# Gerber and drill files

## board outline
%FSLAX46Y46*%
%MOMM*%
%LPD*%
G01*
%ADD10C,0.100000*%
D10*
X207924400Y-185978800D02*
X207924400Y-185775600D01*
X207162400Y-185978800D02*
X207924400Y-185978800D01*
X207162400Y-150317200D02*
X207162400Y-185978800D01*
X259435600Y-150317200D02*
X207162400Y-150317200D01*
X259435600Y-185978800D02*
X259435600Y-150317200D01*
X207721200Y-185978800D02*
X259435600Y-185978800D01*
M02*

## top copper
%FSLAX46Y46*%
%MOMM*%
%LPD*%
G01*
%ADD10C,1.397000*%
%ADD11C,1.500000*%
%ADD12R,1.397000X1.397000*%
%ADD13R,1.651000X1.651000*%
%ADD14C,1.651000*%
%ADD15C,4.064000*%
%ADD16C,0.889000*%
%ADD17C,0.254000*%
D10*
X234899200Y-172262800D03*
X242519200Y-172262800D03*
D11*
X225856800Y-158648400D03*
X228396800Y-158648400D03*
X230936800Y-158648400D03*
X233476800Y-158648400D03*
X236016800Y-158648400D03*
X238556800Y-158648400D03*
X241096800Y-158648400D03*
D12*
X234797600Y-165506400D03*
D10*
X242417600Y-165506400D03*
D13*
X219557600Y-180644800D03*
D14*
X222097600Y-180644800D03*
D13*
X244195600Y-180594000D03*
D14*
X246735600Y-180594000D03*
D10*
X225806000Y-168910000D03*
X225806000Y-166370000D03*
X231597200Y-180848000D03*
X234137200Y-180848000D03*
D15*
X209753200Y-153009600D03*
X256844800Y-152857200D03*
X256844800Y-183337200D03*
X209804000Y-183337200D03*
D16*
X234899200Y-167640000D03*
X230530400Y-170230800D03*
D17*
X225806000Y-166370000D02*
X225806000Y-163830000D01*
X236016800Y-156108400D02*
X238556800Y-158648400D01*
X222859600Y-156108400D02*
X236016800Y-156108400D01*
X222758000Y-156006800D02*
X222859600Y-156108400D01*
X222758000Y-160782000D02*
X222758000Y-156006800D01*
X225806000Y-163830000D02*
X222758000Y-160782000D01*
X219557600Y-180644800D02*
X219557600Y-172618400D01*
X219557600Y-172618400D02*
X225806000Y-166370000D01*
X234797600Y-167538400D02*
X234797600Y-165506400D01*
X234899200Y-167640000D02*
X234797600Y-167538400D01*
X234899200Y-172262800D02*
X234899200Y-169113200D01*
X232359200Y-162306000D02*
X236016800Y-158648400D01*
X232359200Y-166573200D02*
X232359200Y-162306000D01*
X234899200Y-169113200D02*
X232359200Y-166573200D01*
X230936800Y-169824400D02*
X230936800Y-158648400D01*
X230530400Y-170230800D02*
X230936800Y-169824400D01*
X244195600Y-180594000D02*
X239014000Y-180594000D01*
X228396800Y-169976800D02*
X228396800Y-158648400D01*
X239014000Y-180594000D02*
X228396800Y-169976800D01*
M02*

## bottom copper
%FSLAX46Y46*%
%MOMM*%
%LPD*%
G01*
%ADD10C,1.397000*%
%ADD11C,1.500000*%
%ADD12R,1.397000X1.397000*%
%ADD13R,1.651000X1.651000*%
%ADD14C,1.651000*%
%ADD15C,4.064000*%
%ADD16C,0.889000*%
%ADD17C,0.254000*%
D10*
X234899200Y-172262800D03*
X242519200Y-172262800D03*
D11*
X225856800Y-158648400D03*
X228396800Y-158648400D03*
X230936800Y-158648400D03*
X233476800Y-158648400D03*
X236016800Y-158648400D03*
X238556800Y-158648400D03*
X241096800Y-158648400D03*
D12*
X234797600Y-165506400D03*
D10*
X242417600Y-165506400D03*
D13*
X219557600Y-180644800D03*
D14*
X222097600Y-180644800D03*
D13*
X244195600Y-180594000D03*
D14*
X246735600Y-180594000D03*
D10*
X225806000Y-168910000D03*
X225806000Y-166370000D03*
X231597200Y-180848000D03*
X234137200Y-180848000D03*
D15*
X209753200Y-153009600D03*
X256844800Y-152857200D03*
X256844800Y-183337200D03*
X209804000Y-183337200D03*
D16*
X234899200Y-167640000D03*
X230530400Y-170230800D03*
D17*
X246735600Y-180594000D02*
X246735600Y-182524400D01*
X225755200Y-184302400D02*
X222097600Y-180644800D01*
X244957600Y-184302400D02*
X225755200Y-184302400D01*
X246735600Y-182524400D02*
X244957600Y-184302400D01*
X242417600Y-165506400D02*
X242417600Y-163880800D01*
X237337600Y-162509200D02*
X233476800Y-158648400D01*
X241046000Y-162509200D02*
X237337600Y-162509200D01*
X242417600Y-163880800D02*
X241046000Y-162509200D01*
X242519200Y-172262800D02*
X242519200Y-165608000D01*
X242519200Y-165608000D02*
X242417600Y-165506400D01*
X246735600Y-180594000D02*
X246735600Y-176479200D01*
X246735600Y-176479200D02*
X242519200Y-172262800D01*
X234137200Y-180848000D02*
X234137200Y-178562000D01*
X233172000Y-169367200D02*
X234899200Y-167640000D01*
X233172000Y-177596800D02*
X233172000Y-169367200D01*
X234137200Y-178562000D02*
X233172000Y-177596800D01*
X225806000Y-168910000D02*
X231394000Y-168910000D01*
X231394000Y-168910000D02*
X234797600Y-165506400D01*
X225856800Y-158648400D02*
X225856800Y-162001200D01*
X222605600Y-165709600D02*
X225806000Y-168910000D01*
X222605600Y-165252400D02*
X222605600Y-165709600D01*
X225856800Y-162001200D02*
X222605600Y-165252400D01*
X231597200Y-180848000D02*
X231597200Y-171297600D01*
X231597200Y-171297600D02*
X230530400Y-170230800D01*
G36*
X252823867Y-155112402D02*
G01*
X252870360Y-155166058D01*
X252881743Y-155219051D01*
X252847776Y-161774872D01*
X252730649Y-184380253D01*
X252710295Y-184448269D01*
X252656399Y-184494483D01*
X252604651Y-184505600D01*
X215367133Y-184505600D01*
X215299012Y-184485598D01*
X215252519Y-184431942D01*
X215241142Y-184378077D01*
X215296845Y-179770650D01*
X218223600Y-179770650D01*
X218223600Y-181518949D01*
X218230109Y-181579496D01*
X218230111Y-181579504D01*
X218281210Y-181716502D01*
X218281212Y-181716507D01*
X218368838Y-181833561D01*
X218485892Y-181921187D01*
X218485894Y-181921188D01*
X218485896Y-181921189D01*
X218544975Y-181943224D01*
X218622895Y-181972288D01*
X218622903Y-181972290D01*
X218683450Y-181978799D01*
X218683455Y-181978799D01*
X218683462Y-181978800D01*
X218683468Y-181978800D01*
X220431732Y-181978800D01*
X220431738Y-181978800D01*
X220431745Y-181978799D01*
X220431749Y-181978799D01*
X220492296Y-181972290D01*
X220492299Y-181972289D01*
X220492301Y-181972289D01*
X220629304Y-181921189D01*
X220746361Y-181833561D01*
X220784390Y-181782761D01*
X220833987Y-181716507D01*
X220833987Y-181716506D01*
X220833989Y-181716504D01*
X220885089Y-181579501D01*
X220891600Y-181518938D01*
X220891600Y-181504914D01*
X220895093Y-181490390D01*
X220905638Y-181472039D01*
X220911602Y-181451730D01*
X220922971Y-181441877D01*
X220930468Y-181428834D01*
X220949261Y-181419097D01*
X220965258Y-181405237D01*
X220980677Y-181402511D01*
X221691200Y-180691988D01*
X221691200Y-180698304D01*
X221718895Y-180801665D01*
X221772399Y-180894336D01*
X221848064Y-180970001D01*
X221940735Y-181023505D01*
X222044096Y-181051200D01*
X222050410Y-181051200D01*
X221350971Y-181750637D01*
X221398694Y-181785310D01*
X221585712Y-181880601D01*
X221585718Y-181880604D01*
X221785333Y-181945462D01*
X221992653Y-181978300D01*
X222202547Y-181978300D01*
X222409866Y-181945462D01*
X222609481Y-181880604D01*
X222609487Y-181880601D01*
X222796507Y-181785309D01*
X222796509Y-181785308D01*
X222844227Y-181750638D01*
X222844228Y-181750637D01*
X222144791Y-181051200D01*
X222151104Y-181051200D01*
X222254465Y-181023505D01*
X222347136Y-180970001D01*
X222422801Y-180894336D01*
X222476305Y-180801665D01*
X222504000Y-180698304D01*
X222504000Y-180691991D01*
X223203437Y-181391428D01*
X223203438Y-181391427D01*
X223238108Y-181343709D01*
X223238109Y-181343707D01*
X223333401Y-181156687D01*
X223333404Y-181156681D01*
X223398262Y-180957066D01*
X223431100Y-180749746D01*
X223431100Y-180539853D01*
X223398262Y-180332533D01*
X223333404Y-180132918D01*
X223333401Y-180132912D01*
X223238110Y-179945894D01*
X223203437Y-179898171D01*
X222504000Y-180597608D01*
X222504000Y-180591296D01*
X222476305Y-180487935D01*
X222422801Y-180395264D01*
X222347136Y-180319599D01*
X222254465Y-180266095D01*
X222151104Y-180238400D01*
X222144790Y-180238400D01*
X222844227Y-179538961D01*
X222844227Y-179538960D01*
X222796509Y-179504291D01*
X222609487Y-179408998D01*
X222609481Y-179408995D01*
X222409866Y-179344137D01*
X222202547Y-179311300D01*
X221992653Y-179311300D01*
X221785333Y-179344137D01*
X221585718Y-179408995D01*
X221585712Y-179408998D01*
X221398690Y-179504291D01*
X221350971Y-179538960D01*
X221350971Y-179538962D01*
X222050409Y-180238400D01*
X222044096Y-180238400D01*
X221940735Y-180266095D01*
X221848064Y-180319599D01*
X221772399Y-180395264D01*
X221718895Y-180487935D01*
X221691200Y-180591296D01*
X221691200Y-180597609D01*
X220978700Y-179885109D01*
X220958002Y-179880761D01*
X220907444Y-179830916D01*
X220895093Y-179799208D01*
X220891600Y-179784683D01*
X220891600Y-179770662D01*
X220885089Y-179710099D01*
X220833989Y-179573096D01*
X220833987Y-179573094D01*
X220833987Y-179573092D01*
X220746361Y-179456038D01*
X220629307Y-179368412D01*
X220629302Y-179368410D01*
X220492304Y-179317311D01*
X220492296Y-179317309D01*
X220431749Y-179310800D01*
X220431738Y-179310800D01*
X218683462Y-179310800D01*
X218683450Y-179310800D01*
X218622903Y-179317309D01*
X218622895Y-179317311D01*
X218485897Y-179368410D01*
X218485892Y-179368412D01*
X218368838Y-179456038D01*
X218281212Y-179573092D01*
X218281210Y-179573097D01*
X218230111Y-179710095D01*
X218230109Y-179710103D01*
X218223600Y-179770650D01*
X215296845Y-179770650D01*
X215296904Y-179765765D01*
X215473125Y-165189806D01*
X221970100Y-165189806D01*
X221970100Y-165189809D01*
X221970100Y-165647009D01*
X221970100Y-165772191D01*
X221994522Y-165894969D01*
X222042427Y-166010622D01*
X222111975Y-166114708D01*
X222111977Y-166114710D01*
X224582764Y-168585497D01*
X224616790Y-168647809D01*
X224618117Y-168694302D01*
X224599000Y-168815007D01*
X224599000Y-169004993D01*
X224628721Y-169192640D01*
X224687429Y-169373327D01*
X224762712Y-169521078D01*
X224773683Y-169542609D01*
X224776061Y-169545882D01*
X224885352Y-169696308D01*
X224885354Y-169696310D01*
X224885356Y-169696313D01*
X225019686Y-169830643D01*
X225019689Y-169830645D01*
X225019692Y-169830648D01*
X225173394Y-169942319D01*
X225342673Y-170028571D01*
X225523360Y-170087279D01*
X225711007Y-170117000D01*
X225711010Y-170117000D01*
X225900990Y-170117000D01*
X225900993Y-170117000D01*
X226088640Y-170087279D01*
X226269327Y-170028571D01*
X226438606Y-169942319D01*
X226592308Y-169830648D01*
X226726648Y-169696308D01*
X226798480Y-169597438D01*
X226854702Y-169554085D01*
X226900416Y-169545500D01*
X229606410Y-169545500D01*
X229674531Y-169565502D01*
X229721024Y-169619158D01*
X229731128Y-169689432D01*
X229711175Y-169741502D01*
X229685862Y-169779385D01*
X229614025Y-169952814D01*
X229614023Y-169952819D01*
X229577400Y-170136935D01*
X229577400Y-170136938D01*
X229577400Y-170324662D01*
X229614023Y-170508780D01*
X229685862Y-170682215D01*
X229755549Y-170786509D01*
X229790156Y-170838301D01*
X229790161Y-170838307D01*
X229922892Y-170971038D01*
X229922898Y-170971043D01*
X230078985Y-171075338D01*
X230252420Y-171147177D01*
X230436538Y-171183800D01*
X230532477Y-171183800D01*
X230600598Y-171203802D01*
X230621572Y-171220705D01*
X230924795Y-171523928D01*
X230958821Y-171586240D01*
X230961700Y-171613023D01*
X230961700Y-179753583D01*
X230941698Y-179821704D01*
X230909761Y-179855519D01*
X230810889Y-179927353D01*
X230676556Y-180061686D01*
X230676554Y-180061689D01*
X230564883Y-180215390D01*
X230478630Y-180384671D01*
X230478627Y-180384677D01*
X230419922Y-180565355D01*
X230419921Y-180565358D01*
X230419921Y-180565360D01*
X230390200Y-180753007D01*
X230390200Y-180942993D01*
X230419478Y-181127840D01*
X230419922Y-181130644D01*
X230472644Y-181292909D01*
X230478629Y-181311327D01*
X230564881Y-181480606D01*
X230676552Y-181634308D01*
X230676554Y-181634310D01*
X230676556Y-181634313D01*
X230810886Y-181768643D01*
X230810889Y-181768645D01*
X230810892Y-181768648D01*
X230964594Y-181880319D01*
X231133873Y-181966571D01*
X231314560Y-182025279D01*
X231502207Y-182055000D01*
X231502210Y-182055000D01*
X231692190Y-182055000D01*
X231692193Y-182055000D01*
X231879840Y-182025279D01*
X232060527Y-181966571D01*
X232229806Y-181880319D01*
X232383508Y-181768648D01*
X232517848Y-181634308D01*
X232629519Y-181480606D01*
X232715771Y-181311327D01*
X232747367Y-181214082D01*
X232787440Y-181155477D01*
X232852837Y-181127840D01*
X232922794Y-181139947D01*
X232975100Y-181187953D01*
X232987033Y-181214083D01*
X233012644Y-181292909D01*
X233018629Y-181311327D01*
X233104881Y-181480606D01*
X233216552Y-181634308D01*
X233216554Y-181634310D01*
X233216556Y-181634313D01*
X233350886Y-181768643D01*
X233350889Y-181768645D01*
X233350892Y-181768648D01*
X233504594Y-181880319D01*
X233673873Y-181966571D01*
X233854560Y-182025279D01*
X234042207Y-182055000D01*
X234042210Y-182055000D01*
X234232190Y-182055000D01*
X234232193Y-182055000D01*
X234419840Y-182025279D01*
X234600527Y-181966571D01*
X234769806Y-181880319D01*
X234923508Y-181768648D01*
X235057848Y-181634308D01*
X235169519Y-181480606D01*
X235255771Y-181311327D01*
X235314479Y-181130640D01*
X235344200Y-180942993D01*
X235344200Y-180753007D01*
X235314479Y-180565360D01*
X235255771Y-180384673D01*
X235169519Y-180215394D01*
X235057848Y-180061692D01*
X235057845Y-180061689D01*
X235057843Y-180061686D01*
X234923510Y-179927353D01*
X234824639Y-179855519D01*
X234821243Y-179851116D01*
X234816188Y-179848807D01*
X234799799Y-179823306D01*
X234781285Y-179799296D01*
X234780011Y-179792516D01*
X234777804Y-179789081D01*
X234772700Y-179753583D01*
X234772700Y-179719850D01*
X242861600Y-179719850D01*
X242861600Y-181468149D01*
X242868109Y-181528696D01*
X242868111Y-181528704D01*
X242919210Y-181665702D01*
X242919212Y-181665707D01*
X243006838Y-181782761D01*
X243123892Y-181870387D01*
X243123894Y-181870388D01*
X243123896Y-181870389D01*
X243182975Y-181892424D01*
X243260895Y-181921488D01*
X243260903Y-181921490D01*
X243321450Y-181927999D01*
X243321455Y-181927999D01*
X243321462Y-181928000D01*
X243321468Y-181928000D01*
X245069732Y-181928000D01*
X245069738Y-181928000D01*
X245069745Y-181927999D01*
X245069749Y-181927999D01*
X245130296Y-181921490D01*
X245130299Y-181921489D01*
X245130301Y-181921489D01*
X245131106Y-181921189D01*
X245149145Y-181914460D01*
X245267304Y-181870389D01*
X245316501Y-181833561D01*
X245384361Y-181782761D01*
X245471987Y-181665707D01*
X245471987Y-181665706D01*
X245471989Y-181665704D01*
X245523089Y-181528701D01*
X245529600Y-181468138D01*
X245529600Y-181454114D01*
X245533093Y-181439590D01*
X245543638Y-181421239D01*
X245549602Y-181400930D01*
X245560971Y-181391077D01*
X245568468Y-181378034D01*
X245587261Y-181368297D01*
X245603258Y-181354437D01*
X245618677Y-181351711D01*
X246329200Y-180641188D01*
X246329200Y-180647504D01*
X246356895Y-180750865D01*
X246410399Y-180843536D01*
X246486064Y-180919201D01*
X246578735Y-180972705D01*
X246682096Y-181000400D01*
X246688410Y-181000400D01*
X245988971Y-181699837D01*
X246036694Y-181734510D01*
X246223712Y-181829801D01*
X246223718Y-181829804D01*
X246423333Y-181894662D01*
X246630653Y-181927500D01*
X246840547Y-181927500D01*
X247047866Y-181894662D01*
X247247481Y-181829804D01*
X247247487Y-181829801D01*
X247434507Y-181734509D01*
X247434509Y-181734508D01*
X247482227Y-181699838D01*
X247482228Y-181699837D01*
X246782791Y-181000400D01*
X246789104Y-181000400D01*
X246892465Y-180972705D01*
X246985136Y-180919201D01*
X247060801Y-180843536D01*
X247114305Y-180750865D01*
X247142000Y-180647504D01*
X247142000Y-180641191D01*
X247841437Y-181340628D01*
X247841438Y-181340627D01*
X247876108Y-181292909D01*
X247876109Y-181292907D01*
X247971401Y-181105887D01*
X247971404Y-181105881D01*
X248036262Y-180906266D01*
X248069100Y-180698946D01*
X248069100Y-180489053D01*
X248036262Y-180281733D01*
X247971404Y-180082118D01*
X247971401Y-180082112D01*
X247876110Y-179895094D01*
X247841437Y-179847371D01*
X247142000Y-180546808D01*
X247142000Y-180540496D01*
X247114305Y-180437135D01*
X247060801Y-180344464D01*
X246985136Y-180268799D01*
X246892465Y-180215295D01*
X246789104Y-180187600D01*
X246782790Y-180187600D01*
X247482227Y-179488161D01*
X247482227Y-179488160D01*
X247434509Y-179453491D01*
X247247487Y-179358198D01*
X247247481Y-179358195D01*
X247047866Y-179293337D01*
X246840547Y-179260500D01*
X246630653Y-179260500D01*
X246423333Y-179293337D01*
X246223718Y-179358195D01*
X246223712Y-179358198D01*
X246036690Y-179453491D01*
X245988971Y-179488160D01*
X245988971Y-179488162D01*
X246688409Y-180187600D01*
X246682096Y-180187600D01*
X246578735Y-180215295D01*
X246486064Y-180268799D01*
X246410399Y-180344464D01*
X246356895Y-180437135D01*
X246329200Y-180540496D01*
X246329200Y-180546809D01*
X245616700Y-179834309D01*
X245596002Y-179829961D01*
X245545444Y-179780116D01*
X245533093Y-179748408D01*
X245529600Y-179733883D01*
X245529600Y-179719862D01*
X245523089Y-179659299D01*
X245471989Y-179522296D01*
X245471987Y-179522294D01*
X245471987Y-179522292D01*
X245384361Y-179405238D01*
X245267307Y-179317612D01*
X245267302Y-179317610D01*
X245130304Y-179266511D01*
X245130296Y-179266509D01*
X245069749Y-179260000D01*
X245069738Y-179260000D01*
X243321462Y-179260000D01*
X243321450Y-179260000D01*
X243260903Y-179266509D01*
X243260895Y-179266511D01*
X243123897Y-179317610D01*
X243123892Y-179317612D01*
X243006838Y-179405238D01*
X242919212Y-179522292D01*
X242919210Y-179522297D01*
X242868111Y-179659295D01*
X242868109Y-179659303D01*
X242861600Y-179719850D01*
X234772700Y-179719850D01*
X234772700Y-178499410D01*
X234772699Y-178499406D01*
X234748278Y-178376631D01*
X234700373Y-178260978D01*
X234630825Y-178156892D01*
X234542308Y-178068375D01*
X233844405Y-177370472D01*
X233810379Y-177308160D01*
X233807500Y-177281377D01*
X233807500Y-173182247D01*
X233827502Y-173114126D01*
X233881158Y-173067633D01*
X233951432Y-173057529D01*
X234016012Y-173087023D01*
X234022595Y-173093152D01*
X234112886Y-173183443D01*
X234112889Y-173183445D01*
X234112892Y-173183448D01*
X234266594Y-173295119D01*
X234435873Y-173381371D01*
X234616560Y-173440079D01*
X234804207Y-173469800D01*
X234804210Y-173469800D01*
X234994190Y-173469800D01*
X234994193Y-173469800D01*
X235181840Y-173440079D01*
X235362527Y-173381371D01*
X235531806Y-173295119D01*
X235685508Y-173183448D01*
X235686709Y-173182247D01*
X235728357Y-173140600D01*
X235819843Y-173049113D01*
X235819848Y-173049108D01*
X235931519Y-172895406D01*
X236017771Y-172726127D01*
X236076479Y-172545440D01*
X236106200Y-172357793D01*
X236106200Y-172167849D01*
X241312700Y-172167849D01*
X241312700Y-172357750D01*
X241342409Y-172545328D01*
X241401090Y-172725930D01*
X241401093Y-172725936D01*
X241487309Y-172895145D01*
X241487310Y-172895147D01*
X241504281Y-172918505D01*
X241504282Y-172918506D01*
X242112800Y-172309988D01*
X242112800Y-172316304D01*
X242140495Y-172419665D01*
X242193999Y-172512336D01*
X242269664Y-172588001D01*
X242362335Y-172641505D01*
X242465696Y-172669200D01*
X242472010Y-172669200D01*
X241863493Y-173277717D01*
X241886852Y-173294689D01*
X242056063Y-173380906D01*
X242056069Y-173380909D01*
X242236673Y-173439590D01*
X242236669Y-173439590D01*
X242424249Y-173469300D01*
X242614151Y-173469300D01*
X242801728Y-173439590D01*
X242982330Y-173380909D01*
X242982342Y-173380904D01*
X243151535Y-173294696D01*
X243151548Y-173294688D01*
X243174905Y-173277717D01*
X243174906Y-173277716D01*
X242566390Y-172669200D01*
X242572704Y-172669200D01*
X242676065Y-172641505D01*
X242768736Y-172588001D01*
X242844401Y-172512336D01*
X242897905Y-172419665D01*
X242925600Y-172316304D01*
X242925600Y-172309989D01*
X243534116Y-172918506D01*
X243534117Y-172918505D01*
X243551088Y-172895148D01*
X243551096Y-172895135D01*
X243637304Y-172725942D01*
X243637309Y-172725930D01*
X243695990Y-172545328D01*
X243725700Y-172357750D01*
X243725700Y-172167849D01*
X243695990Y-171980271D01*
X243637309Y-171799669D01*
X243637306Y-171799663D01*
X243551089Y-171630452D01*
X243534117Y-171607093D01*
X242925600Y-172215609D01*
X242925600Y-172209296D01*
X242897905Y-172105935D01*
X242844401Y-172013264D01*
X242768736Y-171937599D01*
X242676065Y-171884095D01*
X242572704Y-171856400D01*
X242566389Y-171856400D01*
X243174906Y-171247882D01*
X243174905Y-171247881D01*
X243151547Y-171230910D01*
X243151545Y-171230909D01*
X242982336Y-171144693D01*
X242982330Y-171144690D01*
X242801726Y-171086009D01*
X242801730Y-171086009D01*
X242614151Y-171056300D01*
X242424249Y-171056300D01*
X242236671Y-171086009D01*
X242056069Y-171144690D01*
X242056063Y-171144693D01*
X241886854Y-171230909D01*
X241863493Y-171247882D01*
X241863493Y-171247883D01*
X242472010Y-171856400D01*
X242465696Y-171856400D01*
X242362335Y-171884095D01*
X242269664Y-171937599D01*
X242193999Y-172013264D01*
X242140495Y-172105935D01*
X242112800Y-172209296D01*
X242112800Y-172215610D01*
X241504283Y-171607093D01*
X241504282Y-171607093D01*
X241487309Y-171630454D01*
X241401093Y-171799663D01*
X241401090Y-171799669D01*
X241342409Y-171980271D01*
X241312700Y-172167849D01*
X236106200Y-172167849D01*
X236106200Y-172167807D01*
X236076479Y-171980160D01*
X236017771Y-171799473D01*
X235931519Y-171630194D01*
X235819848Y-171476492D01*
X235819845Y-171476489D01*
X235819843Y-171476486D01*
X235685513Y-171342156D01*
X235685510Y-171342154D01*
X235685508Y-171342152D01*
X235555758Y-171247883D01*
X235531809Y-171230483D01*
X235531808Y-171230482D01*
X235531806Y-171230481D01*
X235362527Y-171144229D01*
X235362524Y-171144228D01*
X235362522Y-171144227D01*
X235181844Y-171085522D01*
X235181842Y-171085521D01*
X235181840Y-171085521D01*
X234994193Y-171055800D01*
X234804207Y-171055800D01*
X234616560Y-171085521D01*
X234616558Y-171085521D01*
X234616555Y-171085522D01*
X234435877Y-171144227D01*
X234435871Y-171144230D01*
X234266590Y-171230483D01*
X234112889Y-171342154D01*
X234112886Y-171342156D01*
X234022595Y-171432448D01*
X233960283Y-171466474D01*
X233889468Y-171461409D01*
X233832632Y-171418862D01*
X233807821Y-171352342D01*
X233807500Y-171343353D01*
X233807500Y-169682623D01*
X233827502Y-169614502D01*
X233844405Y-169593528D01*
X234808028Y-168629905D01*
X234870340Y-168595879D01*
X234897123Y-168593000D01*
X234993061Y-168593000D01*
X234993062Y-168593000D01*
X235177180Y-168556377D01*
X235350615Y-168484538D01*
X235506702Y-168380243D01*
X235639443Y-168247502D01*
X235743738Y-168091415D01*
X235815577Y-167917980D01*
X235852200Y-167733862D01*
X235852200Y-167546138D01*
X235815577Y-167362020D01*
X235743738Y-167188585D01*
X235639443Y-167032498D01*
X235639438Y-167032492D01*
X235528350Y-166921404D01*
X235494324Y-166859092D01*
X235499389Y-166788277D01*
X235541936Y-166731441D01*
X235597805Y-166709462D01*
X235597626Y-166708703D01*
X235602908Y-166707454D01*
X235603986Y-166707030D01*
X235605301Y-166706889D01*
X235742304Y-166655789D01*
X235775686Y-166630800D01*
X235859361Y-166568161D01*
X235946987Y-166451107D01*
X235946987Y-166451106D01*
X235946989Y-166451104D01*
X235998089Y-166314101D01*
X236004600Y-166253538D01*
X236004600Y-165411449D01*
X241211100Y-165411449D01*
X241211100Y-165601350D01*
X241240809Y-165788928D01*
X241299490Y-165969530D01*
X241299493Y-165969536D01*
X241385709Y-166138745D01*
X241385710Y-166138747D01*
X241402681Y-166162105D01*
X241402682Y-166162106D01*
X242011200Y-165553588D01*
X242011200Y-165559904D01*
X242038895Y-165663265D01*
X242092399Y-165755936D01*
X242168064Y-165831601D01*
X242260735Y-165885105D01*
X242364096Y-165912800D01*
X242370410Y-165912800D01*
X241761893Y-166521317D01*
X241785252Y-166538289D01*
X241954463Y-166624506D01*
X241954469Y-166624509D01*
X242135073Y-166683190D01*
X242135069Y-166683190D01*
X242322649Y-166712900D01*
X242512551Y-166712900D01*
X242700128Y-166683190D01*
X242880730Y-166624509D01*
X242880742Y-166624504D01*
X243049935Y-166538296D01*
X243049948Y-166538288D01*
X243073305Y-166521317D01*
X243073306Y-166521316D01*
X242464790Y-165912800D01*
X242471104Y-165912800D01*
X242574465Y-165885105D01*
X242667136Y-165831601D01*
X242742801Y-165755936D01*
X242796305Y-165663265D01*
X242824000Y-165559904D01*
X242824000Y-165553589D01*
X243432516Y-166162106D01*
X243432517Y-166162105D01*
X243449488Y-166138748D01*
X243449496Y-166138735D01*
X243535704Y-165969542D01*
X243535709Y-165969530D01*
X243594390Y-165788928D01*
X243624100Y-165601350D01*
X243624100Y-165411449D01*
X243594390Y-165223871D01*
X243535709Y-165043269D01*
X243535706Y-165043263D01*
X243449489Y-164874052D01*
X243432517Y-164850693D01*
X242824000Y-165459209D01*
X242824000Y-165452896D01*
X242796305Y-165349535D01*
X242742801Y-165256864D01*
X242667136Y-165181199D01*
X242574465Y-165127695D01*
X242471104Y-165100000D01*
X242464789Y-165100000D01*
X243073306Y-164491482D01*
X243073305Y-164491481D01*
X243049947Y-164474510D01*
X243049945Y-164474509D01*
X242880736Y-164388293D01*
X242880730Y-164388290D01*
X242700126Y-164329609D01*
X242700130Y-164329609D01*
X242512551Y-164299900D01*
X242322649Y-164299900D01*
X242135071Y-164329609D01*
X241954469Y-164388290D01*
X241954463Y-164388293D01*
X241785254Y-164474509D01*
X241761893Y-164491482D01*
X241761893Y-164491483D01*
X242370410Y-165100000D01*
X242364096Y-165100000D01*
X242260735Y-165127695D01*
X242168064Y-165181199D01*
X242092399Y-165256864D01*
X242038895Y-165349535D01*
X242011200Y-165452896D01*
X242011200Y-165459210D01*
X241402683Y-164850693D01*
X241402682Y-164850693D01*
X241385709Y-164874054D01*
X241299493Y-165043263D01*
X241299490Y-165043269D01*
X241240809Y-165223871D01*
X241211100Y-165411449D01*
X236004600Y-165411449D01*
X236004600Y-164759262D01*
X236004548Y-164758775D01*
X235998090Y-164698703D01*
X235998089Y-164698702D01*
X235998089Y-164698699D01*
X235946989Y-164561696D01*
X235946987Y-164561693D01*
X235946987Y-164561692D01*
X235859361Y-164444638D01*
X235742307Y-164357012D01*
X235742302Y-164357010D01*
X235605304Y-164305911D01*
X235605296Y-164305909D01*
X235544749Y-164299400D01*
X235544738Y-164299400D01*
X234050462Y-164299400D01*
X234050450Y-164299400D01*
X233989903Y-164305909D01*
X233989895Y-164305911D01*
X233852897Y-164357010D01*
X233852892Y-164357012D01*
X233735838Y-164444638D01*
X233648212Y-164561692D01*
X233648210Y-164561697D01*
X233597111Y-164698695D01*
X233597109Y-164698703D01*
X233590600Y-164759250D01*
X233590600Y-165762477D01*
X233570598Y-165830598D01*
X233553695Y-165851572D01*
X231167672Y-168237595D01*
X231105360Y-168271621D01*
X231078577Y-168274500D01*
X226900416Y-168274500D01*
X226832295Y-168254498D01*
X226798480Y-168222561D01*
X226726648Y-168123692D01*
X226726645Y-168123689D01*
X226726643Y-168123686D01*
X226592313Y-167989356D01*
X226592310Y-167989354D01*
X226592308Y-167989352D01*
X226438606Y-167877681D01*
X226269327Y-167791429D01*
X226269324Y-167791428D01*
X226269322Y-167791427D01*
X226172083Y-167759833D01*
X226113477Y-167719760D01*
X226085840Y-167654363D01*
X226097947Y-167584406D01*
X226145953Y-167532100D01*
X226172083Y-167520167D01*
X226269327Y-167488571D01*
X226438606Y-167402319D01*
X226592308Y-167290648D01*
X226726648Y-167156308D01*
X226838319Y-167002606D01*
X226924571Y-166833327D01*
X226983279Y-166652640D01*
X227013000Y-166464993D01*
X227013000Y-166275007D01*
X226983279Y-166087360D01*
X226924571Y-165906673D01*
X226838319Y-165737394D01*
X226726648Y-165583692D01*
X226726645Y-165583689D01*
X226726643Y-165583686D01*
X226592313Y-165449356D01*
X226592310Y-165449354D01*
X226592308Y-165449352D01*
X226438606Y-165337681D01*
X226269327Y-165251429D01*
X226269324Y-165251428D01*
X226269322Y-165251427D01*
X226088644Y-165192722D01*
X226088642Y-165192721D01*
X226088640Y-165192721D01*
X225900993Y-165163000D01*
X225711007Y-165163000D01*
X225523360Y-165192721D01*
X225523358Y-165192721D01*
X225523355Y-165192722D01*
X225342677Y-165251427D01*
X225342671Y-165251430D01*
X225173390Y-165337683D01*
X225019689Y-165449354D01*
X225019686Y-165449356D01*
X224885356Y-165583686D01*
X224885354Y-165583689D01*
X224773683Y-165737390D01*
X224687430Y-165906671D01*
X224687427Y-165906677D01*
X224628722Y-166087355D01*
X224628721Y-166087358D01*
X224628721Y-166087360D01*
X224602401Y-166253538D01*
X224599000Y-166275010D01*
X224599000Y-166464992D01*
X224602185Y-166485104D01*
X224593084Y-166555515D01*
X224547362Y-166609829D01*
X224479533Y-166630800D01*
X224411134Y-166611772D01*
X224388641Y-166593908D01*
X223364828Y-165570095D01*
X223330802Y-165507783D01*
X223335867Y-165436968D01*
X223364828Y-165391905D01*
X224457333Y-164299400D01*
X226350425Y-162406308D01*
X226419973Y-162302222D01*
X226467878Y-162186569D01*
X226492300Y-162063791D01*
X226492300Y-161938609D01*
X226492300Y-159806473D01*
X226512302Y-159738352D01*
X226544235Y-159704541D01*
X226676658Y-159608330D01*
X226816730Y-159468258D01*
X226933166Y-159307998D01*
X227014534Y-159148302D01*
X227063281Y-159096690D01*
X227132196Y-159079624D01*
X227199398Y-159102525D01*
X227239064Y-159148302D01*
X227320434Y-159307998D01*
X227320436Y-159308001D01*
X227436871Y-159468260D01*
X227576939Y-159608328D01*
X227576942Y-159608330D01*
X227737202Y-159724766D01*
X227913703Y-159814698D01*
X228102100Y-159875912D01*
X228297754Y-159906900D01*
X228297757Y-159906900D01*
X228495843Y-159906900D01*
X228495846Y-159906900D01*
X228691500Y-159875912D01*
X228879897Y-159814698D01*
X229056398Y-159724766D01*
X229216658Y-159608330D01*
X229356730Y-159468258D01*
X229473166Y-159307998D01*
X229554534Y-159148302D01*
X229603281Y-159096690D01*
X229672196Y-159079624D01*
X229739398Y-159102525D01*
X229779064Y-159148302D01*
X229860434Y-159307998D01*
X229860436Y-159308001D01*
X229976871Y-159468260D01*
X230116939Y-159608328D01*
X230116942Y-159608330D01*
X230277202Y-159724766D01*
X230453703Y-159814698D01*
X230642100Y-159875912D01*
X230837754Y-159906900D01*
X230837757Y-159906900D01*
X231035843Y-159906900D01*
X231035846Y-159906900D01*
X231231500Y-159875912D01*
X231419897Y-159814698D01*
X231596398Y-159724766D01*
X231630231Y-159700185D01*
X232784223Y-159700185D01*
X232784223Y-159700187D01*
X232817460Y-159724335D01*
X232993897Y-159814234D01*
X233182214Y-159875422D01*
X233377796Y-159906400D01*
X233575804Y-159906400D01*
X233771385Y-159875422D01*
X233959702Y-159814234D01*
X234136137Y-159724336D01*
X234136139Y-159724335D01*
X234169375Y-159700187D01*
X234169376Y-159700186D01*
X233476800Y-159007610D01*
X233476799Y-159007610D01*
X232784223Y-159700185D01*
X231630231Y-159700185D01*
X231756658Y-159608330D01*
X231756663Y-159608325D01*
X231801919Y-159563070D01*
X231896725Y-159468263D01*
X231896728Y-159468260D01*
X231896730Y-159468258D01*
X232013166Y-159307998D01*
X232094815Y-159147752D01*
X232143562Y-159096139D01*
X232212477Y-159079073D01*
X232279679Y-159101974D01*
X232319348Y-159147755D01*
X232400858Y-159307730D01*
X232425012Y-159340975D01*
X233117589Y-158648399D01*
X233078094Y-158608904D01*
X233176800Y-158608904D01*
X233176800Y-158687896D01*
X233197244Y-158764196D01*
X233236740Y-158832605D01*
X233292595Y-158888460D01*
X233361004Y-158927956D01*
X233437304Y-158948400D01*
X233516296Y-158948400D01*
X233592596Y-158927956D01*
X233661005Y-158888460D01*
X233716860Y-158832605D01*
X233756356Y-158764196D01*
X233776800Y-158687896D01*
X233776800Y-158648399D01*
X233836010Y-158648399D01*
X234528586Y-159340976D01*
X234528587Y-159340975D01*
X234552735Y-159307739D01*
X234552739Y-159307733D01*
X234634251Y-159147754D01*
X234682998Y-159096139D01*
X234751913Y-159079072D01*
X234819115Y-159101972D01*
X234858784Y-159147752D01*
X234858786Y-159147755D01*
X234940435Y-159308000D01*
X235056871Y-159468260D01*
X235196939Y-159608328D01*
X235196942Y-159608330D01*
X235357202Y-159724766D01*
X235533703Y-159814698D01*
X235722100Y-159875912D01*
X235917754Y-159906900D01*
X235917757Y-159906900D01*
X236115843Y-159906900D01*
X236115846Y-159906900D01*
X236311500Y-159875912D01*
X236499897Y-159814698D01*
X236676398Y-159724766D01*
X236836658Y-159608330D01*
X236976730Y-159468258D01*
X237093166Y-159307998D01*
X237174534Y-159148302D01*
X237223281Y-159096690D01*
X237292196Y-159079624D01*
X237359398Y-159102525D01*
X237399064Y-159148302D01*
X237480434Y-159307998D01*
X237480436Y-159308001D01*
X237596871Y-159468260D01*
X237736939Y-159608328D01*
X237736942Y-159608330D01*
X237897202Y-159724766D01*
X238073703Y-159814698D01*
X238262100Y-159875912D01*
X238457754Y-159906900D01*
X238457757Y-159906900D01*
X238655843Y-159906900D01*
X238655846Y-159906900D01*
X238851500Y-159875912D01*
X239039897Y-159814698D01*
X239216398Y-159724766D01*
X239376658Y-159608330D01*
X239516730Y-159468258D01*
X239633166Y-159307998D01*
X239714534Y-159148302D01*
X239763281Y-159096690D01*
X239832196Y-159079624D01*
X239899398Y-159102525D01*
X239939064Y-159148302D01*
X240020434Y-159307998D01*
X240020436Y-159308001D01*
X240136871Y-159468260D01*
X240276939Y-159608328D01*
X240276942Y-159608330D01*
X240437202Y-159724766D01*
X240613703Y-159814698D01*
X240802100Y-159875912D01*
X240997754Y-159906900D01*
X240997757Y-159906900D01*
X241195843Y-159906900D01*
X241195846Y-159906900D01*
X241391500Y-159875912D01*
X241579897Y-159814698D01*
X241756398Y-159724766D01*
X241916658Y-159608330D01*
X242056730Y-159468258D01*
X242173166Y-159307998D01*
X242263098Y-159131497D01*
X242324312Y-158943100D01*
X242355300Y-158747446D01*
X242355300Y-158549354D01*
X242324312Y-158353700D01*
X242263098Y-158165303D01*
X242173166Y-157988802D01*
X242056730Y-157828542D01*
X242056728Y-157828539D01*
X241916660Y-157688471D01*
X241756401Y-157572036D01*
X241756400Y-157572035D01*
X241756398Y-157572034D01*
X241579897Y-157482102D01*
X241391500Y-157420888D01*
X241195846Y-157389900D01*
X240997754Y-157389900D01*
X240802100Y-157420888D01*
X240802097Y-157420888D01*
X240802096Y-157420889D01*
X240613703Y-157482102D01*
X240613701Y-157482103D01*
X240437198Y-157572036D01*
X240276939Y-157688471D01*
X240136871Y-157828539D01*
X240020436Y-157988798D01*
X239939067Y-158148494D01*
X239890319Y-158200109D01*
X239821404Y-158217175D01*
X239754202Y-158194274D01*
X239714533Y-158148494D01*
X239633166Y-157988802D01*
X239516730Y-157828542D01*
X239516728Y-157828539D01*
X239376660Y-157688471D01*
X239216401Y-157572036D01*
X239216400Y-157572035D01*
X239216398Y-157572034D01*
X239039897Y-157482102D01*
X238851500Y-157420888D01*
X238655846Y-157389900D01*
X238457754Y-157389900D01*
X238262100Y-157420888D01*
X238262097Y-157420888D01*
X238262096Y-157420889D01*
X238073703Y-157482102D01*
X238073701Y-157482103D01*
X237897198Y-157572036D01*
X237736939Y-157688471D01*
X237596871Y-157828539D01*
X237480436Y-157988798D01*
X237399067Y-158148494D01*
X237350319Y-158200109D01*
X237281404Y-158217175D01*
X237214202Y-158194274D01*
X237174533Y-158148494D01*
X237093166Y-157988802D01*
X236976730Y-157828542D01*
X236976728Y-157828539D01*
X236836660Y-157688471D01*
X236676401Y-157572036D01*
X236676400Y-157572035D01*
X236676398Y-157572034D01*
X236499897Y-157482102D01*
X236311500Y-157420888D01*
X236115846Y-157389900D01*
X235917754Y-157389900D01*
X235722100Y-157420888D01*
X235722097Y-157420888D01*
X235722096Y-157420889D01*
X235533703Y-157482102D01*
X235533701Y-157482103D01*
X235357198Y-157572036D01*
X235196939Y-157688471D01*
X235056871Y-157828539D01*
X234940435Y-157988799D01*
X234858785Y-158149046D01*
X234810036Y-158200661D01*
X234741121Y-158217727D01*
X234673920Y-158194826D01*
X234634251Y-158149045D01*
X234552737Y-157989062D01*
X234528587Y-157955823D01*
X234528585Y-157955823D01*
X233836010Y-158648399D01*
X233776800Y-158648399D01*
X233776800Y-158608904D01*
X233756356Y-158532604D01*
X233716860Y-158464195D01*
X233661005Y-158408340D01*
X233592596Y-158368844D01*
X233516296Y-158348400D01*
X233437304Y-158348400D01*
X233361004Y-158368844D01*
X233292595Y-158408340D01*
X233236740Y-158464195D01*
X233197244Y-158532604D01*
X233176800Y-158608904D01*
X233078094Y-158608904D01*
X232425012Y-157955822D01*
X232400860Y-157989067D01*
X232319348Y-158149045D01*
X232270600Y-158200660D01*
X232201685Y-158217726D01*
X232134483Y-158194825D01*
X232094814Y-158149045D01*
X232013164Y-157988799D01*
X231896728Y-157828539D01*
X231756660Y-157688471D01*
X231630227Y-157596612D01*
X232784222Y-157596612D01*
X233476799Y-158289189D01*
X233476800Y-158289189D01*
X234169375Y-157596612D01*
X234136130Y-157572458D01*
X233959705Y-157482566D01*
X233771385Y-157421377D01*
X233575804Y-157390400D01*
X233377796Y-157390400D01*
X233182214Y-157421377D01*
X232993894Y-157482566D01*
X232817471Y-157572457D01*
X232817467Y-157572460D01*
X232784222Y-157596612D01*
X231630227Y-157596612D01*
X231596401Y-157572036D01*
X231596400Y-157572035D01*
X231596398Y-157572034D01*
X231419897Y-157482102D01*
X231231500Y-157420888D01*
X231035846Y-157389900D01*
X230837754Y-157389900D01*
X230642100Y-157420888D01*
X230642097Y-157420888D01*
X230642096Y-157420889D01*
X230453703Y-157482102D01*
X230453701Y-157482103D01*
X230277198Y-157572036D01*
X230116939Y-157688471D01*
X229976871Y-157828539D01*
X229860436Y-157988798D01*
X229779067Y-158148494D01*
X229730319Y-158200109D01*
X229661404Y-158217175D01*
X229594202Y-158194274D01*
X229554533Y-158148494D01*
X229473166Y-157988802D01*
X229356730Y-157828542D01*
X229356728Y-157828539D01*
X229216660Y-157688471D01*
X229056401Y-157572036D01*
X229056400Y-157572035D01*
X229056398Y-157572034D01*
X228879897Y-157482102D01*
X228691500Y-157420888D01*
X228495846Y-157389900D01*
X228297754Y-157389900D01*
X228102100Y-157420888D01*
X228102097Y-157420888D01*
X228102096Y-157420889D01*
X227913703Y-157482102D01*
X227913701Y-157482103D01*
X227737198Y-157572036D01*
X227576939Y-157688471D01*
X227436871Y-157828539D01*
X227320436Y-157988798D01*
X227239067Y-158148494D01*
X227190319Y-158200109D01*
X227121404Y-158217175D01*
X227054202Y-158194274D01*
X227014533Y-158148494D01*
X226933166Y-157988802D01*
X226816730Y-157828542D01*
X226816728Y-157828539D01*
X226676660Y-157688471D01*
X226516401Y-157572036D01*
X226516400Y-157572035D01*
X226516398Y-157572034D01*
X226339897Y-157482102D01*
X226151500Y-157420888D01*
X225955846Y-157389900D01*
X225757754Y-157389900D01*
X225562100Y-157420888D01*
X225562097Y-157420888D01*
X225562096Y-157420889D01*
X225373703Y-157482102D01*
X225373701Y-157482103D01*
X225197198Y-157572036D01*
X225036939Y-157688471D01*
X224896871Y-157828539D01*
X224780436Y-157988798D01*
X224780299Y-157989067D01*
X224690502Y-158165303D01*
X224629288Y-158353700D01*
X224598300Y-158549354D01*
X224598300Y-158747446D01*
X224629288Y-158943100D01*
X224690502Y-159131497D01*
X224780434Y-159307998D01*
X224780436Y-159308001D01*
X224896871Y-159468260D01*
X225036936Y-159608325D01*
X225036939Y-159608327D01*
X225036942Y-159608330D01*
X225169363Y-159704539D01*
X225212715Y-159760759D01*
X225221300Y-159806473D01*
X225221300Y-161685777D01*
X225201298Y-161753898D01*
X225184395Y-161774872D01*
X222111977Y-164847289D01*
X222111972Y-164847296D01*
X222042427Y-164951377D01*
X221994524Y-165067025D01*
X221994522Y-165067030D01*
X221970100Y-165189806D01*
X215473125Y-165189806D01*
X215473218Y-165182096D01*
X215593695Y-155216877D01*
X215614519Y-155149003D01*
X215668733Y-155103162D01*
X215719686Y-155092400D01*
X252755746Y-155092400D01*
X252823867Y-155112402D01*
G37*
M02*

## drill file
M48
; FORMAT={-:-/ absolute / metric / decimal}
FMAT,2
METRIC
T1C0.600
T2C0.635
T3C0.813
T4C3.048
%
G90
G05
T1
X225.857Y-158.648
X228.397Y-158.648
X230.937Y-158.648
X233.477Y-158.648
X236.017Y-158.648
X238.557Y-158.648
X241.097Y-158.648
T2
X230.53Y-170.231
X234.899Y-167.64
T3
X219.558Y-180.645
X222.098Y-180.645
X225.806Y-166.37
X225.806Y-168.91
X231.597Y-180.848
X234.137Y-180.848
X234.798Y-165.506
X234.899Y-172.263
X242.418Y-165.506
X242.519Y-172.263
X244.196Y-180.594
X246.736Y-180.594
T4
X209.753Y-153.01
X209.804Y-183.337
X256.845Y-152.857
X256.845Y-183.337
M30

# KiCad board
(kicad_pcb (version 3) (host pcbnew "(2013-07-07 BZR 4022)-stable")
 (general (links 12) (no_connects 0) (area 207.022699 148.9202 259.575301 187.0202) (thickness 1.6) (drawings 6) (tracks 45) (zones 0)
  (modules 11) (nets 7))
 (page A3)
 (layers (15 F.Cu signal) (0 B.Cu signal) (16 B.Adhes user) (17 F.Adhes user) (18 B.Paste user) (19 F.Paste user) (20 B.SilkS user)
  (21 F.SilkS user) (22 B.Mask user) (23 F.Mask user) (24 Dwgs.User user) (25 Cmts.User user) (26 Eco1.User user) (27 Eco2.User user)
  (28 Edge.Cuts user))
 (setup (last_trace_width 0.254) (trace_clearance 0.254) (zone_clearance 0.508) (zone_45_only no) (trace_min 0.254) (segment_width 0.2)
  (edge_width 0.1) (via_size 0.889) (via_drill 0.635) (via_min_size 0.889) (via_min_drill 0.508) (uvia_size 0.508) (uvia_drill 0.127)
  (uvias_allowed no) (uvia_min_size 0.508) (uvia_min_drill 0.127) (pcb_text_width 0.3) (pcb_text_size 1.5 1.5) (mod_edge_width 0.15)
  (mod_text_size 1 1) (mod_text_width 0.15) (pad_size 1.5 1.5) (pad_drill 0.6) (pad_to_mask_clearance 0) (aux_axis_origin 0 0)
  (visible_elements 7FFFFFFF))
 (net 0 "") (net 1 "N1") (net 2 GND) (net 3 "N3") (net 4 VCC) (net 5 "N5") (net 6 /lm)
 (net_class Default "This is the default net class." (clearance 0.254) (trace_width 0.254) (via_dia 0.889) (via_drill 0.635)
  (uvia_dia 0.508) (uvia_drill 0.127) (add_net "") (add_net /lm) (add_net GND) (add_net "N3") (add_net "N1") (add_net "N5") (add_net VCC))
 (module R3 (layer F.Cu) (at 238.7092 172.2628) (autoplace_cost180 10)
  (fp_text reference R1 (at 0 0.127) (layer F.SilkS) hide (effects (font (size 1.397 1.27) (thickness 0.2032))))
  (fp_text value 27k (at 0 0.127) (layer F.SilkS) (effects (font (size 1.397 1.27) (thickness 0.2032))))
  (pad 1 thru_hole circle (at -3.81 0) (size 1.397 1.397) (drill 0.8128) (layers *.Cu *.Mask F.SilkS) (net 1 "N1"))
  (pad 2 thru_hole circle (at 3.81 0) (size 1.397 1.397) (drill 0.8128) (layers *.Cu *.Mask F.SilkS) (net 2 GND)))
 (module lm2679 (layer F.Cu) (at 233.4768 159.9184)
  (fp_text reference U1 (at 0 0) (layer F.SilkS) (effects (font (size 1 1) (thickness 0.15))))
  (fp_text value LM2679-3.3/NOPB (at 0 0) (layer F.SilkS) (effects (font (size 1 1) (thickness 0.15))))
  (pad 1 thru_hole circle (at -7.62 -1.27) (size 1.5 1.5) (drill 0.6) (layers *.Cu *.Mask F.SilkS) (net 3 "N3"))
  (pad 2 thru_hole circle (at -5.08 -1.27) (size 1.5 1.5) (drill 0.6) (layers *.Cu *.Mask F.SilkS) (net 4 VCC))
  (pad 3 thru_hole circle (at -2.54 -1.27) (size 1.5 1.5) (drill 0.6) (layers *.Cu *.Mask F.SilkS) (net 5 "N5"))
  (pad 4 thru_hole circle (at 0 -1.27) (size 1.5 1.5) (drill 0.6) (layers *.Cu *.Mask F.SilkS) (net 2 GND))
  (pad 5 thru_hole circle (at 2.54 -1.27) (size 1.5 1.5) (drill 0.6) (layers *.Cu *.Mask F.SilkS) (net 1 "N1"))
  (pad 6 thru_hole circle (at 5.08 -1.27) (size 1.5 1.5) (drill 0.6) (layers *.Cu *.Mask F.SilkS) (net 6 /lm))
  (pad 7 thru_hole circle (at 7.62 -1.27) (size 1.5 1.5) (drill 0.6) (layers *.Cu *.Mask F.SilkS)))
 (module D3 (layer F.Cu) (at 238.6076 165.5064 180)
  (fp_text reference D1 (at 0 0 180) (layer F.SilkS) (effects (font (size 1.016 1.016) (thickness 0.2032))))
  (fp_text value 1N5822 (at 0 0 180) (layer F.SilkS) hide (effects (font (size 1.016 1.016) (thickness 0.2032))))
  (pad 2 thru_hole rect (at 3.81 0 180) (size 1.397 1.397) (drill 0.8128) (layers *.Cu *.Mask F.SilkS) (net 3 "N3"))
  (pad 1 thru_hole circle (at -3.81 0 180) (size 1.397 1.397) (drill 0.8128) (layers *.Cu *.Mask F.SilkS) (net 2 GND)))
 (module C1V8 (layer F.Cu) (at 220.8276 180.6448)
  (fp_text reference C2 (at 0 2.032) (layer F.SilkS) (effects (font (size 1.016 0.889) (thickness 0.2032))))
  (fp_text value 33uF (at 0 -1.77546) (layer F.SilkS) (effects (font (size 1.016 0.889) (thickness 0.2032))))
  (pad 1 thru_hole rect (at -1.27 0) (size 1.651 1.651) (drill 0.8128) (layers *.Cu *.Mask F.SilkS) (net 6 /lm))
  (pad 2 thru_hole circle (at 1.27 0) (size 1.651 1.651) (drill 0.8128) (layers *.Cu *.Mask F.SilkS) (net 2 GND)))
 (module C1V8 (layer F.Cu) (at 245.4656 180.594)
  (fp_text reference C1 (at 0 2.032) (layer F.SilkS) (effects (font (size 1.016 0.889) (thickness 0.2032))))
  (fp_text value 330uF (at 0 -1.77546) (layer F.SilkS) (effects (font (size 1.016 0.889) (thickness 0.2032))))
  (pad 1 thru_hole rect (at -1.27 0) (size 1.651 1.651) (drill 0.8128) (layers *.Cu *.Mask F.SilkS) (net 4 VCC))
  (pad 2 thru_hole circle (at 1.27 0) (size 1.651 1.651) (drill 0.8128) (layers *.Cu *.Mask F.SilkS) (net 2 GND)))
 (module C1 (layer F.Cu) (at 225.806 167.64 90)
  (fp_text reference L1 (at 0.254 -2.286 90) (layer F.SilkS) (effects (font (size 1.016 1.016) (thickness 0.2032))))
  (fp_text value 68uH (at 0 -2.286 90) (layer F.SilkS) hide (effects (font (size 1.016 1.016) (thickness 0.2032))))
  (pad 1 thru_hole circle (at -1.27 0 90) (size 1.397 1.397) (drill 0.8128) (layers *.Cu *.Mask F.SilkS) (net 3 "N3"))
  (pad 2 thru_hole circle (at 1.27 0 90) (size 1.397 1.397) (drill 0.8128) (layers *.Cu *.Mask F.SilkS) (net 6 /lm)))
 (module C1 (layer F.Cu) (at 232.8672 180.848)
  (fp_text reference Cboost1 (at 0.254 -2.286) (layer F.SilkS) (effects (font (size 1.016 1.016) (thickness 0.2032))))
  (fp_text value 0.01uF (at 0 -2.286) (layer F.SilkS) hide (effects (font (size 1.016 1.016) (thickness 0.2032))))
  (pad 1 thru_hole circle (at -1.27 0) (size 1.397 1.397) (drill 0.8128) (layers *.Cu *.Mask F.SilkS) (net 5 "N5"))
  (pad 2 thru_hole circle (at 1.27 0) (size 1.397 1.397) (drill 0.8128) (layers *.Cu *.Mask F.SilkS) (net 3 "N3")))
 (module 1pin (layer F.Cu) (at 209.7532 153.0096)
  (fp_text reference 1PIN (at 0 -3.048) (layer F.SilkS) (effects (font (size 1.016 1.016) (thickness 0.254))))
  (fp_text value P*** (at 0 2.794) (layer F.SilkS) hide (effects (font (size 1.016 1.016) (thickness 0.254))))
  (pad 1 thru_hole circle (at 0 0) (size 4.064 4.064) (drill 3.048) (layers *.Cu *.Mask F.SilkS)))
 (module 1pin (layer F.Cu) (at 256.8448 152.8572)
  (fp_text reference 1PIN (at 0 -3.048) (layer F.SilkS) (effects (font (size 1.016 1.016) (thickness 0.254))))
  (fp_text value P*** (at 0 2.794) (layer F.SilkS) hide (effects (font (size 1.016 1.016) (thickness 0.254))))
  (pad 1 thru_hole circle (at 0 0) (size 4.064 4.064) (drill 3.048) (layers *.Cu *.Mask F.SilkS)))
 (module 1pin (layer F.Cu) (at 256.8448 183.3372)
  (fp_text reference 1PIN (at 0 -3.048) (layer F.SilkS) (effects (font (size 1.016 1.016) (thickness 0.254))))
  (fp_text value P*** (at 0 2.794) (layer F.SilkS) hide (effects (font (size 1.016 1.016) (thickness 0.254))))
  (pad 1 thru_hole circle (at 0 0) (size 4.064 4.064) (drill 3.048) (layers *.Cu *.Mask F.SilkS)))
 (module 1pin (layer F.Cu) (at 209.804 183.3372)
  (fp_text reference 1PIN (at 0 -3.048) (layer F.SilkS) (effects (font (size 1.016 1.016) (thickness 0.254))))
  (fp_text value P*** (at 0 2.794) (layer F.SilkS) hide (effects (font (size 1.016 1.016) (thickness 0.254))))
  (pad 1 thru_hole circle (at 0 0) (size 4.064 4.064) (drill 3.048) (layers *.Cu *.Mask F.SilkS)))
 (gr_line (start 207.9244 185.9788) (end 207.9244 185.7756) (angle 90) (layer Edge.Cuts) (width 0.1))
 (gr_line (start 207.1624 185.9788) (end 207.9244 185.9788) (angle 90) (layer Edge.Cuts) (width 0.1))
 (gr_line (start 207.1624 150.3172) (end 207.1624 185.9788) (angle 90) (layer Edge.Cuts) (width 0.1))
 (gr_line (start 259.4356 150.3172) (end 207.1624 150.3172) (angle 90) (layer Edge.Cuts) (width 0.1))
 (gr_line (start 259.4356 185.9788) (end 259.4356 150.3172) (angle 90) (layer Edge.Cuts) (width 0.1))
 (gr_line (start 207.7212 185.9788) (end 259.4356 185.9788) (angle 90) (layer Edge.Cuts) (width 0.1))
 (segment (start 225.806 166.37) (end 225.806 163.83) (width 0.254) (layer F.Cu) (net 6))
 (segment (start 236.0168 156.1084) (end 238.5568 158.6484) (width 0.254) (layer F.Cu) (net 6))
 (segment (start 222.8596 156.1084) (end 236.0168 156.1084) (width 0.254) (layer F.Cu) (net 6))
 (segment (start 222.758 156.0068) (end 222.8596 156.1084) (width 0.254) (layer F.Cu) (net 6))
 (segment (start 222.758 160.782) (end 222.758 156.0068) (width 0.254) (layer F.Cu) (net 6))
 (segment (start 225.806 163.83) (end 222.758 160.782) (width 0.254) (layer F.Cu) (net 6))
 (segment (start 219.5576 180.6448) (end 219.5576 172.6184) (width 0.254) (layer F.Cu) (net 6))
 (segment (start 219.5576 172.6184) (end 225.806 166.37) (width 0.254) (layer F.Cu) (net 6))
 (segment (start 246.7356 180.594) (end 246.7356 182.5244) (width 0.254) (layer B.Cu) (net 2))
 (segment (start 225.7552 184.3024) (end 222.0976 180.6448) (width 0.254) (layer B.Cu) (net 2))
 (segment (start 244.9576 184.3024) (end 225.7552 184.3024) (width 0.254) (layer B.Cu) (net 2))
 (segment (start 246.7356 182.5244) (end 244.9576 184.3024) (width 0.254) (layer B.Cu) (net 2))
 (segment (start 242.4176 165.5064) (end 242.4176 163.8808) (width 0.254) (layer B.Cu) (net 2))
 (segment (start 237.3376 162.5092) (end 233.4768 158.6484) (width 0.254) (layer B.Cu) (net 2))
 (segment (start 241.046 162.5092) (end 237.3376 162.5092) (width 0.254) (layer B.Cu) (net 2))
 (segment (start 242.4176 163.8808) (end 241.046 162.5092) (width 0.254) (layer B.Cu) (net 2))
 (segment (start 242.5192 172.2628) (end 242.5192 165.608) (width 0.254) (layer B.Cu) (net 2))
 (segment (start 242.5192 165.608) (end 242.4176 165.5064) (width 0.254) (layer B.Cu) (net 2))
 (segment (start 246.7356 180.594) (end 246.7356 176.4792) (width 0.254) (layer B.Cu) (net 2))
 (segment (start 246.7356 176.4792) (end 242.5192 172.2628) (width 0.254) (layer B.Cu) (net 2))
 (segment (start 234.1372 180.848) (end 234.1372 178.562) (width 0.254) (layer B.Cu) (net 3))
 (segment (start 234.7976 167.5384) (end 234.7976 165.5064) (width 0.254) (layer F.Cu) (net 3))
 (segment (start 234.8992 167.64) (end 234.7976 167.5384) (width 0.254) (layer F.Cu) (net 3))
 (via (at 234.8992 167.64) (size 0.889) (layers F.Cu B.Cu) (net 3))
 (segment (start 233.172 169.3672) (end 234.8992 167.64) (width 0.254) (layer B.Cu) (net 3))
 (segment (start 233.172 177.5968) (end 233.172 169.3672) (width 0.254) (layer B.Cu) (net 3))
 (segment (start 234.1372 178.562) (end 233.172 177.5968) (width 0.254) (layer B.Cu) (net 3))
 (segment (start 225.806 168.91) (end 231.394 168.91) (width 0.254) (layer B.Cu) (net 3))
 (segment (start 231.394 168.91) (end 234.7976 165.5064) (width 0.254) (layer B.Cu) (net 3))
 (segment (start 225.8568 158.6484) (end 225.8568 162.0012) (width 0.254) (layer B.Cu) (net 3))
 (segment (start 222.6056 165.7096) (end 225.806 168.91) (width 0.254) (layer B.Cu) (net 3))
 (segment (start 222.6056 165.2524) (end 222.6056 165.7096) (width 0.254) (layer B.Cu) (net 3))
 (segment (start 225.8568 162.0012) (end 222.6056 165.2524) (width 0.254) (layer B.Cu) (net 3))
 (segment (start 234.8992 172.2628) (end 234.8992 169.1132) (width 0.254) (layer F.Cu) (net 1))
 (segment (start 232.3592 162.306) (end 236.0168 158.6484) (width 0.254) (layer F.Cu) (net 1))
 (segment (start 232.3592 166.5732) (end 232.3592 162.306) (width 0.254) (layer F.Cu) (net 1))
 (segment (start 234.8992 169.1132) (end 232.3592 166.5732) (width 0.254) (layer F.Cu) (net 1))
 (segment (start 231.5972 180.848) (end 231.5972 171.2976) (width 0.254) (layer B.Cu) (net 5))
 (segment (start 230.9368 169.8244) (end 230.9368 158.6484) (width 0.254) (layer F.Cu) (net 5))
 (segment (start 230.5304 170.2308) (end 230.9368 169.8244) (width 0.254) (layer F.Cu) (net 5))
 (via (at 230.5304 170.2308) (size 0.889) (layers F.Cu B.Cu) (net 5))
 (segment (start 231.5972 171.2976) (end 230.5304 170.2308) (width 0.254) (layer B.Cu) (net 5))
 (segment (start 244.1956 180.594) (end 239.014 180.594) (width 0.254) (layer F.Cu) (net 4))
 (segment (start 228.3968 169.9768) (end 228.3968 158.6484) (width 0.254) (layer F.Cu) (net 4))
 (segment (start 239.014 180.594) (end 228.3968 169.9768) (width 0.254) (layer F.Cu) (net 4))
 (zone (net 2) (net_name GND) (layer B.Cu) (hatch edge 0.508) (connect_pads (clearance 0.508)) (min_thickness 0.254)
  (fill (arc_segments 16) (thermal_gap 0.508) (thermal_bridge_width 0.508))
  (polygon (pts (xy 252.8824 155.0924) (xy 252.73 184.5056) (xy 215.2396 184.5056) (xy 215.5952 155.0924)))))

